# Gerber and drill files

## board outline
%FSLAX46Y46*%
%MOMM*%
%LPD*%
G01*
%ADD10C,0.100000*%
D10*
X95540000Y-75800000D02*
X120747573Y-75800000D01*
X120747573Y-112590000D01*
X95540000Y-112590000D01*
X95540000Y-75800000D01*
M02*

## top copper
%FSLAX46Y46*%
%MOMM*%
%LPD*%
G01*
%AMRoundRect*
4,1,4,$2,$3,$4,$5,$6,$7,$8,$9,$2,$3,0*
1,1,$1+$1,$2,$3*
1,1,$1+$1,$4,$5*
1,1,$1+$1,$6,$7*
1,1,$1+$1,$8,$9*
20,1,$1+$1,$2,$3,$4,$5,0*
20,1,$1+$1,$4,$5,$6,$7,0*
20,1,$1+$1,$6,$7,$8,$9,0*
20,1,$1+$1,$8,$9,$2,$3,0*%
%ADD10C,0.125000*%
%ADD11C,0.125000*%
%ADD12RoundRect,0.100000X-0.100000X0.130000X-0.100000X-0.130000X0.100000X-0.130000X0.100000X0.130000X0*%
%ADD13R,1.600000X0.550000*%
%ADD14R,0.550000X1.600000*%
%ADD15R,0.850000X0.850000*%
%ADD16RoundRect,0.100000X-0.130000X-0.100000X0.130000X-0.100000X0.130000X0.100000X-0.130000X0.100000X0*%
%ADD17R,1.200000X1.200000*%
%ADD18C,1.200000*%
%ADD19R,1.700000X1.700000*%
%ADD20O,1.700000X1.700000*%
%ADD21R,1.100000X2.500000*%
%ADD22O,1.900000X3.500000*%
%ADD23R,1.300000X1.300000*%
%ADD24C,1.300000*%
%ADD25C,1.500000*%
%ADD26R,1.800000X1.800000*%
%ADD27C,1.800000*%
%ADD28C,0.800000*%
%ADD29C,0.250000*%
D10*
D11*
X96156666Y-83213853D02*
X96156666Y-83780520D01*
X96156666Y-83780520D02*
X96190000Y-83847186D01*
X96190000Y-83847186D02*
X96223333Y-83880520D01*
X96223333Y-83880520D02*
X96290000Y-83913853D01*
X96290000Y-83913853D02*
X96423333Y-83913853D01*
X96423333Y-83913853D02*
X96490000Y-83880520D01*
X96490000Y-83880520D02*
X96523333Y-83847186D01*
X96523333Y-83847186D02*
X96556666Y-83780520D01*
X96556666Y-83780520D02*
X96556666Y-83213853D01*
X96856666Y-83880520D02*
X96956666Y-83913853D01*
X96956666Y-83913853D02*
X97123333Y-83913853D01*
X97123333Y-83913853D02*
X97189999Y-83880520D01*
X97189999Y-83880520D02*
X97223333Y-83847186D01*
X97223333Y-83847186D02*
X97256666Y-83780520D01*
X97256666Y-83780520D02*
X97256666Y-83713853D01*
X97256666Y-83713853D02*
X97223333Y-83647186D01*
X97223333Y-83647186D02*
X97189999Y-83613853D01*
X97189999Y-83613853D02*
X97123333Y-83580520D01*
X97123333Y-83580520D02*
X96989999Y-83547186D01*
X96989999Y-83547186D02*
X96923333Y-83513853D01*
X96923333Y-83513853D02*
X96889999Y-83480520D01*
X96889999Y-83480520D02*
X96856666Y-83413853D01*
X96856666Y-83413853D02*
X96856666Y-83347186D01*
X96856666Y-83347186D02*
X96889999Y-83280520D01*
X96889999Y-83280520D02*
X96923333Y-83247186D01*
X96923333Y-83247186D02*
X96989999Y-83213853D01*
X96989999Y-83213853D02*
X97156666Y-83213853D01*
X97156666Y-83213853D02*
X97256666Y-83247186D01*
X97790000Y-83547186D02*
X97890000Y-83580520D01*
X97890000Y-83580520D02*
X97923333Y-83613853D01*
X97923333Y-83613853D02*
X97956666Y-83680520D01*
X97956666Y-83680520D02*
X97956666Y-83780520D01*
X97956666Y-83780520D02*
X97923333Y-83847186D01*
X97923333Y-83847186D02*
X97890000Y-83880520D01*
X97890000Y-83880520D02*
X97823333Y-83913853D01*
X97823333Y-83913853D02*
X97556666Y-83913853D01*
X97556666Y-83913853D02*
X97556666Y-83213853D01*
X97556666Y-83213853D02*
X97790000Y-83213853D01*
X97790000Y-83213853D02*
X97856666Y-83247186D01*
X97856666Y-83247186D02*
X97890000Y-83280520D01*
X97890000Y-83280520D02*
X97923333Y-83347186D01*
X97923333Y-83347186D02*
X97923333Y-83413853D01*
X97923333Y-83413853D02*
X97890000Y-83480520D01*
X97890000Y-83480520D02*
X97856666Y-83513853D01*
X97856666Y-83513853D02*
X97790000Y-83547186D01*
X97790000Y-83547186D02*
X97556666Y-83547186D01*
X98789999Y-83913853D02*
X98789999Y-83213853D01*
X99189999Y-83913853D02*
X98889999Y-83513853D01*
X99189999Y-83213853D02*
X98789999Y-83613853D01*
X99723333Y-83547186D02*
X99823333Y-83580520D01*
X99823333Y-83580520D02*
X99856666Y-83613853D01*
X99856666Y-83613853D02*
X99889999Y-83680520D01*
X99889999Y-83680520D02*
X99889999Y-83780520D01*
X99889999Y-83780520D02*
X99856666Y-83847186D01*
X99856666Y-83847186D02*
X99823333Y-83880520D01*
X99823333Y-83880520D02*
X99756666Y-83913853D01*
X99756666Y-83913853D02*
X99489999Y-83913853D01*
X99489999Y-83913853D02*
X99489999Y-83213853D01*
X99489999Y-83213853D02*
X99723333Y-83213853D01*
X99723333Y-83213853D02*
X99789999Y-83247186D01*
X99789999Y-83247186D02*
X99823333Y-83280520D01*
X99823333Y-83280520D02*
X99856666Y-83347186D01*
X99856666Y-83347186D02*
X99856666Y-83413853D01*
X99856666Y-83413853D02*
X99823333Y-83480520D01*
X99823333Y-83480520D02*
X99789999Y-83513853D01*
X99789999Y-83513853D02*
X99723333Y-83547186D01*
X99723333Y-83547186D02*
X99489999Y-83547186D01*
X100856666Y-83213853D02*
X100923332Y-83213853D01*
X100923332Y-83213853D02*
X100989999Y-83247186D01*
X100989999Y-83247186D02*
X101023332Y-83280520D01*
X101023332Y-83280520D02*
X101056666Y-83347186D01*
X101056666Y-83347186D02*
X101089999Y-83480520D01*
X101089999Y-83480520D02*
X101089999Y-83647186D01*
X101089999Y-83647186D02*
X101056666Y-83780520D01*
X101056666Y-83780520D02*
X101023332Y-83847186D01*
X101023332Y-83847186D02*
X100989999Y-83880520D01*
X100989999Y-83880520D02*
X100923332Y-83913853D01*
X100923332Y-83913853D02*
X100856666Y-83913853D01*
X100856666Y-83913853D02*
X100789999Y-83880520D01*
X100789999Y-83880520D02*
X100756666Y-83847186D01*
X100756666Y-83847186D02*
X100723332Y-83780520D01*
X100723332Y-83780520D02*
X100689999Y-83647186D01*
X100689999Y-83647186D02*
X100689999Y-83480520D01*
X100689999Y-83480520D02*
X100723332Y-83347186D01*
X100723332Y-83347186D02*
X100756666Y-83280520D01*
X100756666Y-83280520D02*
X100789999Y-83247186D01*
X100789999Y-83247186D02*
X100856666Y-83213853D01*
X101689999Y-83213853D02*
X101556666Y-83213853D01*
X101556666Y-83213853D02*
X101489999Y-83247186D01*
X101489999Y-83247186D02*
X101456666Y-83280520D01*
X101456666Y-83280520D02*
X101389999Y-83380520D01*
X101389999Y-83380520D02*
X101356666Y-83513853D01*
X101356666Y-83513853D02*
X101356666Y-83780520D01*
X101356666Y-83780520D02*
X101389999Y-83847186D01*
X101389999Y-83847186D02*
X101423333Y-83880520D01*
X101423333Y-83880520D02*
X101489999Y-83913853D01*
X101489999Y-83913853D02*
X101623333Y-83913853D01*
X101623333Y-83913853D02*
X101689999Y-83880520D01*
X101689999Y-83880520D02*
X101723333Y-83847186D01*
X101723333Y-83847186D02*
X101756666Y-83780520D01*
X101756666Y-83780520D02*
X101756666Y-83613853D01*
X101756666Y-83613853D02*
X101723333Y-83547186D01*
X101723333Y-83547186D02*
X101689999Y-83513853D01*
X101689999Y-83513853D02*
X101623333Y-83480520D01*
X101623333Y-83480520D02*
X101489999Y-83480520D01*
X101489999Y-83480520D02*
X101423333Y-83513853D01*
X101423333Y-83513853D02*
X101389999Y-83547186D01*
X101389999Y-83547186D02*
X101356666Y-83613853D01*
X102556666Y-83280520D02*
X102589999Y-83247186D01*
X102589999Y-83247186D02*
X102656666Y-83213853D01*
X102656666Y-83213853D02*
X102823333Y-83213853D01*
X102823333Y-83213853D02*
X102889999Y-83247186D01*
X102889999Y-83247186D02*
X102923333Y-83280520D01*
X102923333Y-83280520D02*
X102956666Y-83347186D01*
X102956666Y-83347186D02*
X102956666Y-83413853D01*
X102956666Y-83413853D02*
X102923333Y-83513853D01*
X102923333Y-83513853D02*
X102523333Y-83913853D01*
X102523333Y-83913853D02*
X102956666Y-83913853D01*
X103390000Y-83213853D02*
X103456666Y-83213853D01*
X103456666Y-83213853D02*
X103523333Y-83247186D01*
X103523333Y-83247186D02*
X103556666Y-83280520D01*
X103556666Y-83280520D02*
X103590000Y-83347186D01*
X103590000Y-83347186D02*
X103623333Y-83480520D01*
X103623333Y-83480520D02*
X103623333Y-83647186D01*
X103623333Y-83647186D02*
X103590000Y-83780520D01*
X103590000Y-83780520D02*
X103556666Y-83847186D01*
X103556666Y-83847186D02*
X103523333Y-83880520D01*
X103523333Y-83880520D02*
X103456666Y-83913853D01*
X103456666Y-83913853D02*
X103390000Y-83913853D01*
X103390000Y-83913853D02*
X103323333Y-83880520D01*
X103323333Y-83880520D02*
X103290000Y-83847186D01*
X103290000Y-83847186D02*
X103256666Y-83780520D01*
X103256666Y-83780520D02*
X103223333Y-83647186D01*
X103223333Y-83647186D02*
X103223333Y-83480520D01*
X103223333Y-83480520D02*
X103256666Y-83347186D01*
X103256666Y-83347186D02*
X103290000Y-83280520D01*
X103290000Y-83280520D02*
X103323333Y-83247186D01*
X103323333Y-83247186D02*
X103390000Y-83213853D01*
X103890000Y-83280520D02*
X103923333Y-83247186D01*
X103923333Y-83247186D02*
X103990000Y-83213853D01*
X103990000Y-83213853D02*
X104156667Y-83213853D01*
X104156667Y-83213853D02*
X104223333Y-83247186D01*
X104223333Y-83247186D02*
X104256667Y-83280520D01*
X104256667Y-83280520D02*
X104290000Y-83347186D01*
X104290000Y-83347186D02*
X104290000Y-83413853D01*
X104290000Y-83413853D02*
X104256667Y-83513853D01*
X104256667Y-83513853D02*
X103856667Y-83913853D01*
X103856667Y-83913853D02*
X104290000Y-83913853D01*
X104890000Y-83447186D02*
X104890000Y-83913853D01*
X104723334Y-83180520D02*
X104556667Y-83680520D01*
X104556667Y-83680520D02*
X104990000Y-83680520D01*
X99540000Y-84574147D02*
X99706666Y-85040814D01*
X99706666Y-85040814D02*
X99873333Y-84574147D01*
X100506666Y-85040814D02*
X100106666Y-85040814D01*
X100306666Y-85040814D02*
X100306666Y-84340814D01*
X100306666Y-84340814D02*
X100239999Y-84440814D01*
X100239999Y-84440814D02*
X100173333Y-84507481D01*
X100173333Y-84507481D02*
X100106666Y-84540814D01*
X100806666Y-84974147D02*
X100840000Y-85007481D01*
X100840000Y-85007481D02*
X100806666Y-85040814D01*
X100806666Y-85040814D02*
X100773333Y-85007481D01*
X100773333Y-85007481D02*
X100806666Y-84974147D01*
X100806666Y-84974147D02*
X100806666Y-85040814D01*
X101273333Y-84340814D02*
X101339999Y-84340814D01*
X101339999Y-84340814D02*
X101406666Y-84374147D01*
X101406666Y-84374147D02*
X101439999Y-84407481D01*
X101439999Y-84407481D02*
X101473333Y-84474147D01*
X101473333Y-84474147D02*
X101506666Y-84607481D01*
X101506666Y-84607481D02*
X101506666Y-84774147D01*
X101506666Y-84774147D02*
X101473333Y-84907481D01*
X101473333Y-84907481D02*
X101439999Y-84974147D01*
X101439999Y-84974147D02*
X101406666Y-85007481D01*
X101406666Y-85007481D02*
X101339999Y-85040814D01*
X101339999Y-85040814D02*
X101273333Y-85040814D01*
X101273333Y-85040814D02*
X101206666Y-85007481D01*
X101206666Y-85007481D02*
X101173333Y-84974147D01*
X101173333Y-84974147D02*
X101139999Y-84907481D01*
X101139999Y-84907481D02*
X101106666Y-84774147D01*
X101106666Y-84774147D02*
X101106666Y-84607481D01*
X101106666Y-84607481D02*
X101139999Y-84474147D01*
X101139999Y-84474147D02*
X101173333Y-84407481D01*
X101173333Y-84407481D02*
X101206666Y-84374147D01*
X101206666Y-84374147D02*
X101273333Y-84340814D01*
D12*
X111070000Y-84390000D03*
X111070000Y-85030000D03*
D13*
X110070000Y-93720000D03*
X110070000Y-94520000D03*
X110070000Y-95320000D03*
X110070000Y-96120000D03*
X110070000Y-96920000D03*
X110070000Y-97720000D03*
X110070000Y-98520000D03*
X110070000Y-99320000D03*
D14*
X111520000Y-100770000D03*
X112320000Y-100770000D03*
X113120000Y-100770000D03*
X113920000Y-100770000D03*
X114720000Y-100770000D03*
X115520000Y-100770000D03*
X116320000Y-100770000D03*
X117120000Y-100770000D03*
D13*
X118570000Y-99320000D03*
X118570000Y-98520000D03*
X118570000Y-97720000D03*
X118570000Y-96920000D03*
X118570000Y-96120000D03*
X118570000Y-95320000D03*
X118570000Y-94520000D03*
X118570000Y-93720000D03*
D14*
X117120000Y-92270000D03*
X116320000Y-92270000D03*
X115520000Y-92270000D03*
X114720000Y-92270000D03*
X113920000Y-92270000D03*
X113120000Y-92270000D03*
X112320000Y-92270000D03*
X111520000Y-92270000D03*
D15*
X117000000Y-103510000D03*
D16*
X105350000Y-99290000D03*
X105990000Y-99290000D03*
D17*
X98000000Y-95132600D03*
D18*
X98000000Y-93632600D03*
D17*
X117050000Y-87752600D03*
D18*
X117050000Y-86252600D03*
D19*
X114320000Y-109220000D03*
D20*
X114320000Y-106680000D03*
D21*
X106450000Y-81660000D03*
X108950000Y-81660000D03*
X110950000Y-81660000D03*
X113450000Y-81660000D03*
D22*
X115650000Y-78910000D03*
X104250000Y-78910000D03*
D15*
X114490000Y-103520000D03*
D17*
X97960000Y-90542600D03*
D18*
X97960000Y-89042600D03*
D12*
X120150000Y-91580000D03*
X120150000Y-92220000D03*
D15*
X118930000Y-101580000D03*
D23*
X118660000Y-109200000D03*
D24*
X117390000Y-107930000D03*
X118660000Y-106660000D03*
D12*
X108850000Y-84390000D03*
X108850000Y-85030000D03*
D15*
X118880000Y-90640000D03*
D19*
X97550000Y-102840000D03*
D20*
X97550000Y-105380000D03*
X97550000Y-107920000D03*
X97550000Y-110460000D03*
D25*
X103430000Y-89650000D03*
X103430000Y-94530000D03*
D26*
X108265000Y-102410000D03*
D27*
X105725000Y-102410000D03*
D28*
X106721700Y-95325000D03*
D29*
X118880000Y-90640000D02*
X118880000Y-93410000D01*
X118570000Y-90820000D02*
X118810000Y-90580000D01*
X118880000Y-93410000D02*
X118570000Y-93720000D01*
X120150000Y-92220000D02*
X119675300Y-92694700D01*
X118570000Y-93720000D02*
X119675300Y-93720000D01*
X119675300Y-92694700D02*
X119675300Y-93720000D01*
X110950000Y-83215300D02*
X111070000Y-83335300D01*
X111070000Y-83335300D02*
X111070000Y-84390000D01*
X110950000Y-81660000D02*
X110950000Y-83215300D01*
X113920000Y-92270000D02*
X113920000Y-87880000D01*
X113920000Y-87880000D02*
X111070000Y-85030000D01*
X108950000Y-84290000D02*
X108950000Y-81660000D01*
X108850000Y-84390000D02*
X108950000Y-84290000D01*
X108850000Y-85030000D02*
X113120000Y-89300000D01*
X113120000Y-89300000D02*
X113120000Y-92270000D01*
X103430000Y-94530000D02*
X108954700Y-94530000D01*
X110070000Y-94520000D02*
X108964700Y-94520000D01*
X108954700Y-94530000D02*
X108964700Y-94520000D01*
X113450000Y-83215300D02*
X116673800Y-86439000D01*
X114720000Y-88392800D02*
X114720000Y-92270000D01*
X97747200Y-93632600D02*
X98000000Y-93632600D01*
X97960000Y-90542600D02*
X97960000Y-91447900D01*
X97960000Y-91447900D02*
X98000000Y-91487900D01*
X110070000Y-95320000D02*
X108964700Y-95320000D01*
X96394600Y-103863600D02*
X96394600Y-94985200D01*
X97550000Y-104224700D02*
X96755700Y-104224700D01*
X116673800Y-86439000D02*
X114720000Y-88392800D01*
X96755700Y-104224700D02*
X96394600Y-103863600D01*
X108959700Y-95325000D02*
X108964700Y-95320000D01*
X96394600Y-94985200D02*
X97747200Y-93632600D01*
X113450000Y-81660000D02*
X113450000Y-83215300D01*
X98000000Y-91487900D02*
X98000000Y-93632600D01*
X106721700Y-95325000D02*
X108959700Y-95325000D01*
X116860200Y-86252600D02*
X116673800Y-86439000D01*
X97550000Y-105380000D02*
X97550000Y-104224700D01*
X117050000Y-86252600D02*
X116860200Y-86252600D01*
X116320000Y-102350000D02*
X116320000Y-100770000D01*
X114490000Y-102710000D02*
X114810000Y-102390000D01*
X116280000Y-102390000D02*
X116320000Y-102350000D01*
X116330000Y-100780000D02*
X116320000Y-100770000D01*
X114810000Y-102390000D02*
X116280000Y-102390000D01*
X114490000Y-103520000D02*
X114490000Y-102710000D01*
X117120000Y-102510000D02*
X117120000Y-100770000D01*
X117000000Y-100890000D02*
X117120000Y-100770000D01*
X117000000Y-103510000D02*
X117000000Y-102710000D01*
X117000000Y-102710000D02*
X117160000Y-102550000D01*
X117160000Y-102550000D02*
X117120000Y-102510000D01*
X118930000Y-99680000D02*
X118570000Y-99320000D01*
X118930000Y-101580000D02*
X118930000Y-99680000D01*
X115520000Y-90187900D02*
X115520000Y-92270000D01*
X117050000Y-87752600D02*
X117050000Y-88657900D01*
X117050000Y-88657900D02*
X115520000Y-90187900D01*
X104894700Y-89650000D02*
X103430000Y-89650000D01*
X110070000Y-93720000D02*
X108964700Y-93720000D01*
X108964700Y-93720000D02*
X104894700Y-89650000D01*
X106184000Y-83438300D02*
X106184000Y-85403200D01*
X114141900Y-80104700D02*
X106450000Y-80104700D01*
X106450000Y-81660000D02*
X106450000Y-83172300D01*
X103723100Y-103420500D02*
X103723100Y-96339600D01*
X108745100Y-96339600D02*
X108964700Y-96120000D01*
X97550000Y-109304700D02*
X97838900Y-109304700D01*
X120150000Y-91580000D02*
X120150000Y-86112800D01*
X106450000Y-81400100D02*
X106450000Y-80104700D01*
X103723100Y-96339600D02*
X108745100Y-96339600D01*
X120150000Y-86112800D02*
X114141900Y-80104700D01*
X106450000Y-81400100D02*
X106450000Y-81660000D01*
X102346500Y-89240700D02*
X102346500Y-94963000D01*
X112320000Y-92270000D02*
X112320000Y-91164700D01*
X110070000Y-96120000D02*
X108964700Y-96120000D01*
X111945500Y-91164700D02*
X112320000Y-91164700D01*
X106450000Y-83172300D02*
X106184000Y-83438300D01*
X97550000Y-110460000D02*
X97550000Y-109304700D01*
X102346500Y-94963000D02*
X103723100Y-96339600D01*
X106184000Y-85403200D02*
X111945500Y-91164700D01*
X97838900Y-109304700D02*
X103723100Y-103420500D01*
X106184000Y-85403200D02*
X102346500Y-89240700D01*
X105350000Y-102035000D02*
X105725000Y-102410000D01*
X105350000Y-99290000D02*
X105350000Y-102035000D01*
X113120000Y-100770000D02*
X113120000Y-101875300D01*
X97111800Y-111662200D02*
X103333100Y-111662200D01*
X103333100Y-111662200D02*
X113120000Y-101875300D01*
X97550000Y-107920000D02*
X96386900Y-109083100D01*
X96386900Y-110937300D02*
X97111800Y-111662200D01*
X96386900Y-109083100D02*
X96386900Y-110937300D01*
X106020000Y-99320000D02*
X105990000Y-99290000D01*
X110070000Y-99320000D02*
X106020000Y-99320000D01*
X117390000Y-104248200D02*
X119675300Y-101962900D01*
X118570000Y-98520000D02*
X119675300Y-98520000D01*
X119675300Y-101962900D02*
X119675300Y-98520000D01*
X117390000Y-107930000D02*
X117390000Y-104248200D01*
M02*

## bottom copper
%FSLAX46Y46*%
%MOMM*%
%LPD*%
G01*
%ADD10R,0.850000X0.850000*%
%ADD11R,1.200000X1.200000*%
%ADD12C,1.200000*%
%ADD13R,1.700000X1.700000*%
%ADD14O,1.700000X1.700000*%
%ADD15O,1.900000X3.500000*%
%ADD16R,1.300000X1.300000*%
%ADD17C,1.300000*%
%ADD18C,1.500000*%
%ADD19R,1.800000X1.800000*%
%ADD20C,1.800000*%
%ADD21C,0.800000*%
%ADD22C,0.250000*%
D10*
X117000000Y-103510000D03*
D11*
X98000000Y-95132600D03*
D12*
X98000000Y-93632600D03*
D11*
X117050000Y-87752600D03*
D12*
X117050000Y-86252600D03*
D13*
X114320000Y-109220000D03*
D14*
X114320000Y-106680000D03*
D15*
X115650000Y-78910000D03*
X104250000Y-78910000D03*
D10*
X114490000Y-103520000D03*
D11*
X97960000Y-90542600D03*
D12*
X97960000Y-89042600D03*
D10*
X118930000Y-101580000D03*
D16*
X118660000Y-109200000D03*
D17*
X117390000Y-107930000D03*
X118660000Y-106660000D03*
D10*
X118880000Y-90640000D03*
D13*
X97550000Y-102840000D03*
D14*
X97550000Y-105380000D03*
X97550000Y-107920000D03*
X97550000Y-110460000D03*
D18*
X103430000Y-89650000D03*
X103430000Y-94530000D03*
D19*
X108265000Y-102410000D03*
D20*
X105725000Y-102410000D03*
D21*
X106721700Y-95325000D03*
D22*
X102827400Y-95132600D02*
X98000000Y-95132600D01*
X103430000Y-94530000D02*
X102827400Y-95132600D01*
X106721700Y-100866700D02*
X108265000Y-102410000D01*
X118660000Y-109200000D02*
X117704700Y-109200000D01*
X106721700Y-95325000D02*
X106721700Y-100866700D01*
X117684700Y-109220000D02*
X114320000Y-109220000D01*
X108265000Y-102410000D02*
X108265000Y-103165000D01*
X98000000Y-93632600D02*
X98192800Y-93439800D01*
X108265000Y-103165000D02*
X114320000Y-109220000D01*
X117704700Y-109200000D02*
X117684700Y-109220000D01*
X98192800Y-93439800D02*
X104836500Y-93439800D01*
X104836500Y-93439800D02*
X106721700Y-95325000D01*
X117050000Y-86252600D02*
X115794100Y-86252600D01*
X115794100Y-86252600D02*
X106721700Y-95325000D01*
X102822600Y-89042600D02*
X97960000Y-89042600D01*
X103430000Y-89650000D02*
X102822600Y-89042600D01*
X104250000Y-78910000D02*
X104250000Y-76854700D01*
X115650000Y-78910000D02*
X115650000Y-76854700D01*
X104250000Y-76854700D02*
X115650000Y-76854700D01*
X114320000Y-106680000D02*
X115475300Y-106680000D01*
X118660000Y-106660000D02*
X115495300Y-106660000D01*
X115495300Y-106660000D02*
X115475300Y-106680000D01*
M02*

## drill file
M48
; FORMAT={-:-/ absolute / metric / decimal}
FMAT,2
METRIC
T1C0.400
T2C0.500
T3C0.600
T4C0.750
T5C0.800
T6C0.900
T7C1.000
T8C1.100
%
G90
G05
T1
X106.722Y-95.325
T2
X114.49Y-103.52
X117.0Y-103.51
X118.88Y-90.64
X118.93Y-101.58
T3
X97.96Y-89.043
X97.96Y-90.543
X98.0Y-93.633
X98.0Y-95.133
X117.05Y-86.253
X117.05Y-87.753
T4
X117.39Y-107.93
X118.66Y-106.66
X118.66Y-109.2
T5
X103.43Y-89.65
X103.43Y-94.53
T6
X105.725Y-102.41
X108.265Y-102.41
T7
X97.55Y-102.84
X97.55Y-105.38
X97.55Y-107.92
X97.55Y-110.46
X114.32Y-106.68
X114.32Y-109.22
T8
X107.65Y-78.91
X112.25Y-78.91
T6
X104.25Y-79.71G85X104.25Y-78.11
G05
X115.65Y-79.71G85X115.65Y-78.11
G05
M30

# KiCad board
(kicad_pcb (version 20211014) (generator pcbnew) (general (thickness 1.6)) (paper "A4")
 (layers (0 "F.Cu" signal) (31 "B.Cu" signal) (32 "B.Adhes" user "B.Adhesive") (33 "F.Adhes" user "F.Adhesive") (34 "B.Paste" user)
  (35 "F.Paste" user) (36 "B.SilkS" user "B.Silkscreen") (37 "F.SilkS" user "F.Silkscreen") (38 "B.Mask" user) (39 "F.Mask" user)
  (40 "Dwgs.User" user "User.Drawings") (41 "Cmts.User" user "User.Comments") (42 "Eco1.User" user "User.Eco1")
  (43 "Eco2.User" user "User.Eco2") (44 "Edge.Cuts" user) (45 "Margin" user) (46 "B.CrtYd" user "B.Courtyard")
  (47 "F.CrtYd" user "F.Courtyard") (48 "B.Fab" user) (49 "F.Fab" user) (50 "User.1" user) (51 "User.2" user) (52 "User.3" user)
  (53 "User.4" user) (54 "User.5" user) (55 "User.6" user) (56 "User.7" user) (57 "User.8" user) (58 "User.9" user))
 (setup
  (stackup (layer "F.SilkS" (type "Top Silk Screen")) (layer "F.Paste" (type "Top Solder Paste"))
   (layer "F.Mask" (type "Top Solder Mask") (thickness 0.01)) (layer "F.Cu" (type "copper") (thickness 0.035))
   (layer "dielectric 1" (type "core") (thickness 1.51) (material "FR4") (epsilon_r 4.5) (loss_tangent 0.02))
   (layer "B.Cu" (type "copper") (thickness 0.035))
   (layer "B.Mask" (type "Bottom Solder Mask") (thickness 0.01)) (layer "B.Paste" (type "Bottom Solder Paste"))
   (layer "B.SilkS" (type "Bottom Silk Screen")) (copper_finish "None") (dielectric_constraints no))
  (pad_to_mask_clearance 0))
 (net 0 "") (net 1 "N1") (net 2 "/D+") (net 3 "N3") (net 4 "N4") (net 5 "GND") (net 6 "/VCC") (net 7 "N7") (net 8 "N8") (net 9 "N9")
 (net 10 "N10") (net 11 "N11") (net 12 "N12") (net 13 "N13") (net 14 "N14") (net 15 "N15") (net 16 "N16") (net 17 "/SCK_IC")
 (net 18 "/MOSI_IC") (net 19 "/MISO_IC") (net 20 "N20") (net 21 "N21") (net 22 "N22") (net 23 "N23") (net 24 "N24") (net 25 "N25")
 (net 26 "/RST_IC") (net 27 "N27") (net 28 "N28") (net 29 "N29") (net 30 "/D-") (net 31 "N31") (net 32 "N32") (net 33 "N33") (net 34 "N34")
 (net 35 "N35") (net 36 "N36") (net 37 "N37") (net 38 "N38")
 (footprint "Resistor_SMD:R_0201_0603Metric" (layer "F.Cu") (at 111.07 84.71 -90)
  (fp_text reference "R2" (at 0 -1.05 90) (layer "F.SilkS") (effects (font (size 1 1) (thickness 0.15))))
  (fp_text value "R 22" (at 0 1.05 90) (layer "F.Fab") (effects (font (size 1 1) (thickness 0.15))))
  (pad "" smd roundrect (at 0.345 0 270) (size 0.318 0.36) (layers "F.Paste") (roundrect_rratio 0.25))
  (pad "" smd roundrect (at -0.345 0 270) (size 0.318 0.36) (layers "F.Paste") (roundrect_rratio 0.25))
  (pad "1" smd roundrect (at -0.32 0 270) (size 0.46 0.4) (layers "F.Cu" "F.Mask") (roundrect_rratio 0.25) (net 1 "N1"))
  (pad "2" smd roundrect (at 0.32 0 270) (size 0.46 0.4) (layers "F.Cu" "F.Mask") (roundrect_rratio 0.25) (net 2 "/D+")))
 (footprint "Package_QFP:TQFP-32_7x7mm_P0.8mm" (layer "F.Cu") (at 114.32 96.52)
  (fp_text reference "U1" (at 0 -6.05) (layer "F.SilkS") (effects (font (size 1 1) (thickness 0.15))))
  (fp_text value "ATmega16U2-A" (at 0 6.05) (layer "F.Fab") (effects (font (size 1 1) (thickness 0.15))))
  (pad "1" smd rect (at -4.25 -2.8) (size 1.6 0.55) (layers "F.Cu" "F.Paste" "F.Mask") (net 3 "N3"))
  (pad "2" smd rect (at -4.25 -2) (size 1.6 0.55) (layers "F.Cu" "F.Paste" "F.Mask") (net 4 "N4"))
  (pad "3" smd rect (at -4.25 -1.2) (size 1.6 0.55) (layers "F.Cu" "F.Paste" "F.Mask") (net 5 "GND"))
  (pad "4" smd rect (at -4.25 -0.4) (size 1.6 0.55) (layers "F.Cu" "F.Paste" "F.Mask") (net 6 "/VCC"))
  (pad "5" smd rect (at -4.25 0.4) (size 1.6 0.55) (layers "F.Cu" "F.Paste" "F.Mask") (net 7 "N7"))
  (pad "6" smd rect (at -4.25 1.2) (size 1.6 0.55) (layers "F.Cu" "F.Paste" "F.Mask") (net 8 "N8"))
  (pad "7" smd rect (at -4.25 2) (size 1.6 0.55) (layers "F.Cu" "F.Paste" "F.Mask") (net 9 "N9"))
  (pad "8" smd rect (at -4.25 2.8) (size 1.6 0.55) (layers "F.Cu" "F.Paste" "F.Mask") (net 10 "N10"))
  (pad "9" smd rect (at -2.8 4.25 90) (size 1.6 0.55) (layers "F.Cu" "F.Paste" "F.Mask") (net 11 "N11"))
  (pad "10" smd rect (at -2 4.25 90) (size 1.6 0.55) (layers "F.Cu" "F.Paste" "F.Mask") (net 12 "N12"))
  (pad "11" smd rect (at -1.2 4.25 90) (size 1.6 0.55) (layers "F.Cu" "F.Paste" "F.Mask") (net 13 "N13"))
  (pad "12" smd rect (at -0.4 4.25 90) (size 1.6 0.55) (layers "F.Cu" "F.Paste" "F.Mask") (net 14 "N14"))
  (pad "13" smd rect (at 0.4 4.25 90) (size 1.6 0.55) (layers "F.Cu" "F.Paste" "F.Mask") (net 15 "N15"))
  (pad "14" smd rect (at 1.2 4.25 90) (size 1.6 0.55) (layers "F.Cu" "F.Paste" "F.Mask") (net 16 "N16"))
  (pad "15" smd rect (at 2 4.25 90) (size 1.6 0.55) (layers "F.Cu" "F.Paste" "F.Mask") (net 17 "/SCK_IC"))
  (pad "16" smd rect (at 2.8 4.25 90) (size 1.6 0.55) (layers "F.Cu" "F.Paste" "F.Mask") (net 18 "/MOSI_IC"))
  (pad "17" smd rect (at 4.25 2.8) (size 1.6 0.55) (layers "F.Cu" "F.Paste" "F.Mask") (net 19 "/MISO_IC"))
  (pad "18" smd rect (at 4.25 2) (size 1.6 0.55) (layers "F.Cu" "F.Paste" "F.Mask") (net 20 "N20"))
  (pad "19" smd rect (at 4.25 1.2) (size 1.6 0.55) (layers "F.Cu" "F.Paste" "F.Mask") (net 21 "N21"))
  (pad "20" smd rect (at 4.25 0.4) (size 1.6 0.55) (layers "F.Cu" "F.Paste" "F.Mask") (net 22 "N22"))
  (pad "21" smd rect (at 4.25 -0.4) (size 1.6 0.55) (layers "F.Cu" "F.Paste" "F.Mask") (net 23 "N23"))
  (pad "22" smd rect (at 4.25 -1.2) (size 1.6 0.55) (layers "F.Cu" "F.Paste" "F.Mask") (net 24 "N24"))
  (pad "23" smd rect (at 4.25 -2) (size 1.6 0.55) (layers "F.Cu" "F.Paste" "F.Mask") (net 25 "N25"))
  (pad "24" smd rect (at 4.25 -2.8) (size 1.6 0.55) (layers "F.Cu" "F.Paste" "F.Mask") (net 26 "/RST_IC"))
  (pad "25" smd rect (at 2.8 -4.25 90) (size 1.6 0.55) (layers "F.Cu" "F.Paste" "F.Mask") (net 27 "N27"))
  (pad "26" smd rect (at 2 -4.25 90) (size 1.6 0.55) (layers "F.Cu" "F.Paste" "F.Mask") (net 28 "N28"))
  (pad "27" smd rect (at 1.2 -4.25 90) (size 1.6 0.55) (layers "F.Cu" "F.Paste" "F.Mask") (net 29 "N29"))
  (pad "28" smd rect (at 0.4 -4.25 90) (size 1.6 0.55) (layers "F.Cu" "F.Paste" "F.Mask") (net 5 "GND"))
  (pad "29" smd rect (at -0.4 -4.25 90) (size 1.6 0.55) (layers "F.Cu" "F.Paste" "F.Mask") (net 2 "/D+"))
  (pad "30" smd rect (at -1.2 -4.25 90) (size 1.6 0.55) (layers "F.Cu" "F.Paste" "F.Mask") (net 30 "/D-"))
  (pad "31" smd rect (at -2 -4.25 90) (size 1.6 0.55) (layers "F.Cu" "F.Paste" "F.Mask") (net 6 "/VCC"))
  (pad "32" smd rect (at -2.8 -4.25 90) (size 1.6 0.55) (layers "F.Cu" "F.Paste" "F.Mask") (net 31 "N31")))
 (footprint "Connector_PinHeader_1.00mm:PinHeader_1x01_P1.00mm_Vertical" (layer "F.Cu") (at 117 103.51)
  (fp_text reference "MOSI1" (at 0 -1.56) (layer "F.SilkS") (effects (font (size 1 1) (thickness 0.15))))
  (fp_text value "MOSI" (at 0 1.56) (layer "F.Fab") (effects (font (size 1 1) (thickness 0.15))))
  (pad "1" thru_hole rect (at 0 0) (size 0.85 0.85) (drill 0.5) (layers *.Cu *.Mask) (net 18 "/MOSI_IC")))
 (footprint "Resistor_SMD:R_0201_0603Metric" (layer "F.Cu") (at 105.67 99.29)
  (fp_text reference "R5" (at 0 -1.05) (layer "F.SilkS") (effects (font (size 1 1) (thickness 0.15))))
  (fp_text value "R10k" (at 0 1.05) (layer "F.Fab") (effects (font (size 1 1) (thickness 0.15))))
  (pad "" smd roundrect (at 0.345 0) (size 0.318 0.36) (layers "F.Paste") (roundrect_rratio 0.25))
  (pad "" smd roundrect (at -0.345 0) (size 0.318 0.36) (layers "F.Paste") (roundrect_rratio 0.25))
  (pad "1" smd roundrect (at -0.32 0) (size 0.46 0.4) (layers "F.Cu" "F.Mask") (roundrect_rratio 0.25) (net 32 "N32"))
  (pad "2" smd roundrect (at 0.32 0) (size 0.46 0.4) (layers "F.Cu" "F.Mask") (roundrect_rratio 0.25) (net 10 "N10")))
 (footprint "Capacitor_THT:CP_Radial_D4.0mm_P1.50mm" (layer "F.Cu") (at 98 95.1326 90)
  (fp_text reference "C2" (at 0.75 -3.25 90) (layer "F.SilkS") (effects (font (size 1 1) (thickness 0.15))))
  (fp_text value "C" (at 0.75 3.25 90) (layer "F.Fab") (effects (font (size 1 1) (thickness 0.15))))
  (pad "1" thru_hole rect (at 0 0 90) (size 1.2 1.2) (drill 0.6) (layers *.Cu *.Mask) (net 4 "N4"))
  (pad "2" thru_hole circle (at 1.5 0 90) (size 1.2 1.2) (drill 0.6) (layers *.Cu *.Mask) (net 5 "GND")))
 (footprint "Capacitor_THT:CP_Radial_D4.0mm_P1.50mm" (layer "F.Cu") (at 117.05 87.7526 90)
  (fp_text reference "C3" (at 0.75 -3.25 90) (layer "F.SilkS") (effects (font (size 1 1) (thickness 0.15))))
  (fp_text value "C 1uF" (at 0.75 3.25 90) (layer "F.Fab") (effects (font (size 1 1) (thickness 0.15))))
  (pad "1" thru_hole rect (at 0 0 90) (size 1.2 1.2) (drill 0.6) (layers *.Cu *.Mask) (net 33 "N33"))
  (pad "2" thru_hole circle (at 1.5 0 90) (size 1.2 1.2) (drill 0.6) (layers *.Cu *.Mask) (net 5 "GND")))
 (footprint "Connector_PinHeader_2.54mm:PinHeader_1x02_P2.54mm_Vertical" (layer "F.Cu") (at 114.32 109.22 180)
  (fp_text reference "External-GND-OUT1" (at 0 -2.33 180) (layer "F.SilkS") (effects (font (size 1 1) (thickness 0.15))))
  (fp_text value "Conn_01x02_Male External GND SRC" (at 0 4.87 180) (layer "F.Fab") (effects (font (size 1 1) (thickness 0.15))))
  (pad "1" thru_hole rect (at 0 0 180) (size 1.7 1.7) (drill 1) (layers *.Cu *.Mask) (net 5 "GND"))
  (pad "2" thru_hole oval (at 0 2.54 180) (size 1.7 1.7) (drill 1) (layers *.Cu *.Mask) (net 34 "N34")))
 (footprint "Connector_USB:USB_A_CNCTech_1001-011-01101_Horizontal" (layer "F.Cu") (at 109.95 72.01 90)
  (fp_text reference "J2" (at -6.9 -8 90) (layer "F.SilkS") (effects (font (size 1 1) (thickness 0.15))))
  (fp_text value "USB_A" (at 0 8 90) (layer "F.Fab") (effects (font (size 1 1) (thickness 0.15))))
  (pad "" np_thru_hole circle (at -6.9 2.3 90) (size 1.1 1.1) (drill 1.1) (layers *.Cu *.Mask))
  (pad "" np_thru_hole circle (at -6.9 -2.3 90) (size 1.1 1.1) (drill 1.1) (layers *.Cu *.Mask))
  (pad "1" smd rect (at -9.65 -3.5 90) (size 2.5 1.1) (layers "F.Cu" "F.Paste" "F.Mask") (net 6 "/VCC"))
  (pad "2" smd rect (at -9.65 -1 90) (size 2.5 1.1) (layers "F.Cu" "F.Paste" "F.Mask") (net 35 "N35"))
  (pad "3" smd rect (at -9.65 1 90) (size 2.5 1.1) (layers "F.Cu" "F.Paste" "F.Mask") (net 1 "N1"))
  (pad "4" smd rect (at -9.65 3.5 90) (size 2.5 1.1) (layers "F.Cu" "F.Paste" "F.Mask") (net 5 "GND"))
  (pad "5" thru_hole oval (at -6.9 5.7 90) (size 3.5 1.9) (drill oval 2.5 0.9) (layers *.Cu *.Mask) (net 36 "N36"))
  (pad "5" thru_hole oval (at -6.9 -5.7 90) (size 3.5 1.9) (drill oval 2.5 0.9) (layers *.Cu *.Mask) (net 36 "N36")))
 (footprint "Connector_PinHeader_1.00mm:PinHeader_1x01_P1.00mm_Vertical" (layer "F.Cu") (at 114.49 103.52)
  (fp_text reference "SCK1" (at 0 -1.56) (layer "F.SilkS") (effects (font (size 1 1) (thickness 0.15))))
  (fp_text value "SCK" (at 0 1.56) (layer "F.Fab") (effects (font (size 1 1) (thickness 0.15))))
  (pad "1" thru_hole rect (at 0 0) (size 0.85 0.85) (drill 0.5) (layers *.Cu *.Mask) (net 17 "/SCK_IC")))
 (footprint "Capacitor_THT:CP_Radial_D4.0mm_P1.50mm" (layer "F.Cu") (at 97.96 90.5426 90)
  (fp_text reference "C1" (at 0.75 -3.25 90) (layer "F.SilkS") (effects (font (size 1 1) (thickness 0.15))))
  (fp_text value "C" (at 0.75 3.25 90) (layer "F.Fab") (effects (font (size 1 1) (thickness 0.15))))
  (pad "1" thru_hole rect (at 0 0 90) (size 1.2 1.2) (drill 0.6) (layers *.Cu *.Mask) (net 5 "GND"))
  (pad "2" thru_hole circle (at 1.5 0 90) (size 1.2 1.2) (drill 0.6) (layers *.Cu *.Mask) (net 3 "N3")))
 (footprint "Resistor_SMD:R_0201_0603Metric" (layer "F.Cu") (at 120.15 91.9 -90)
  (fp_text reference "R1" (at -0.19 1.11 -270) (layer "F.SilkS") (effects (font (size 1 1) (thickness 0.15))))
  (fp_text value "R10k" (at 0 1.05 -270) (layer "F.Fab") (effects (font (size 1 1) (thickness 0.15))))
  (pad "" smd roundrect (at -0.345 0 270) (size 0.318 0.36) (layers "F.Paste") (roundrect_rratio 0.25))
  (pad "" smd roundrect (at 0.345 0 270) (size 0.318 0.36) (layers "F.Paste") (roundrect_rratio 0.25))
  (pad "1" smd roundrect (at -0.32 0 270) (size 0.46 0.4) (layers "F.Cu" "F.Mask") (roundrect_rratio 0.25) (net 6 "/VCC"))
  (pad "2" smd roundrect (at 0.32 0 270) (size 0.46 0.4) (layers "F.Cu" "F.Mask") (roundrect_rratio 0.25) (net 26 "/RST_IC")))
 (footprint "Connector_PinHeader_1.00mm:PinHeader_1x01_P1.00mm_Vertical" (layer "F.Cu") (at 118.93 101.58)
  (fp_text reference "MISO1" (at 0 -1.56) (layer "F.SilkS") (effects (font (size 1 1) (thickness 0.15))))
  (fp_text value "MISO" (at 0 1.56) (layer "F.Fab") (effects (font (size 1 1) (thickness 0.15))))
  (pad "1" thru_hole rect (at 0 0) (size 0.85 0.85) (drill 0.5) (layers *.Cu *.Mask) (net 19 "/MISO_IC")))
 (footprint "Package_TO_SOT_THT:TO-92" (layer "F.Cu") (at 118.66 109.2 90)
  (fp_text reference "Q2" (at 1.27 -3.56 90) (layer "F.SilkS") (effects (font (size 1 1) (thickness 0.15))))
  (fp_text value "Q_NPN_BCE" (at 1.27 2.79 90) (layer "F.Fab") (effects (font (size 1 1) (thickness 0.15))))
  (pad "1" thru_hole rect (at 0 0 90) (size 1.3 1.3) (drill 0.75) (layers *.Cu *.Mask) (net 5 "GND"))
  (pad "2" thru_hole circle (at 1.27 -1.27 90) (size 1.3 1.3) (drill 0.75) (layers *.Cu *.Mask) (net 20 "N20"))
  (pad "3" thru_hole circle (at 2.54 0 90) (size 1.3 1.3) (drill 0.75) (layers *.Cu *.Mask) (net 34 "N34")))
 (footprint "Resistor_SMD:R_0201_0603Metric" (layer "F.Cu") (at 108.85 84.71 -90)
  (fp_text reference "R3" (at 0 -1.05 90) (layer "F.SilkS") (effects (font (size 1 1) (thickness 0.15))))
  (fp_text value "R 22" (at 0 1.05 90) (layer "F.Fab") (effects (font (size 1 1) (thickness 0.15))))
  (pad "" smd roundrect (at -0.345 0 270) (size 0.318 0.36) (layers "F.Paste") (roundrect_rratio 0.25))
  (pad "" smd roundrect (at 0.345 0 270) (size 0.318 0.36) (layers "F.Paste") (roundrect_rratio 0.25))
  (pad "1" smd roundrect (at -0.32 0 270) (size 0.46 0.4) (layers "F.Cu" "F.Mask") (roundrect_rratio 0.25) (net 35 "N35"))
  (pad "2" smd roundrect (at 0.32 0 270) (size 0.46 0.4) (layers "F.Cu" "F.Mask") (roundrect_rratio 0.25) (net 30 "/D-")))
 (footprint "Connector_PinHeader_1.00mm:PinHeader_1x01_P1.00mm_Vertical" (layer "F.Cu") (at 118.88 90.64)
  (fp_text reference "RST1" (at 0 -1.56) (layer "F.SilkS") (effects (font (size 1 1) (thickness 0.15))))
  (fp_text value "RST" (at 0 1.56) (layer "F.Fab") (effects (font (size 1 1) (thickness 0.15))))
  (pad "1" thru_hole rect (at 0 0) (size 0.85 0.85) (drill 0.5) (layers *.Cu *.Mask) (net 26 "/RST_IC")))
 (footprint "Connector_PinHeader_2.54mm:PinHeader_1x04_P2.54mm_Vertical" (layer "F.Cu") (at 97.55 102.84)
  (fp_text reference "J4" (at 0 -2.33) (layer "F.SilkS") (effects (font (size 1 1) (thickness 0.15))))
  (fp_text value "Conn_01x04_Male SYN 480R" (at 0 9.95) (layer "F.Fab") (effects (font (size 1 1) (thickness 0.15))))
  (pad "1" thru_hole rect (at 0 0) (size 1.7 1.7) (drill 1) (layers *.Cu *.Mask) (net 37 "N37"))
  (pad "2" thru_hole oval (at 0 2.54) (size 1.7 1.7) (drill 1) (layers *.Cu *.Mask) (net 5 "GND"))
  (pad "3" thru_hole oval (at 0 5.08) (size 1.7 1.7) (drill 1) (layers *.Cu *.Mask) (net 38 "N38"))
  (pad "4" thru_hole oval (at 0 7.62) (size 1.7 1.7) (drill 1) (layers *.Cu *.Mask) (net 6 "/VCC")))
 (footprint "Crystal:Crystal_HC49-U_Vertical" (layer "F.Cu") (at 103.43 89.65 -90)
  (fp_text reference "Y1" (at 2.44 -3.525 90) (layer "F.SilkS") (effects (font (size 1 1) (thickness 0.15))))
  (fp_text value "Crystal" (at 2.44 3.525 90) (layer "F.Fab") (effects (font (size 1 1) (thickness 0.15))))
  (pad "1" thru_hole circle (at 0 0 270) (size 1.5 1.5) (drill 0.8) (layers *.Cu *.Mask) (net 3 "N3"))
  (pad "2" thru_hole circle (at 4.88 0 270) (size 1.5 1.5) (drill 0.8) (layers *.Cu *.Mask) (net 4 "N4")))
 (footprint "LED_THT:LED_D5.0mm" (layer "F.Cu") (at 108.265 102.41 180)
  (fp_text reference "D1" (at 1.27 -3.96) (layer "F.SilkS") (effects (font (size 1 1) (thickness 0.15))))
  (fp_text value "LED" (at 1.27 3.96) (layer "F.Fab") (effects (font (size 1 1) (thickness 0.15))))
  (pad "1" thru_hole rect (at 0 0 180) (size 1.8 1.8) (drill 0.9) (layers *.Cu *.Mask) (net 5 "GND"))
  (pad "2" thru_hole circle (at 2.54 0 180) (size 1.8 1.8) (drill 0.9) (layers *.Cu *.Mask) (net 32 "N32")))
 (gr_rect (start 120.747573 75.8) (end 95.54 112.59) (layer "Edge.Cuts") (width 0.1) (fill none))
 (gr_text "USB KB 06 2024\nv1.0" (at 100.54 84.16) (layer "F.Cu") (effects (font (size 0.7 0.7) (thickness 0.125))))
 (segment (start 118.88 90.64) (end 118.88 93.41) (width 0.25) (layer "F.Cu") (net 26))
 (segment (start 118.57 90.82) (end 118.81 90.58) (width 0.25) (layer "F.Cu") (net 26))
 (segment (start 118.88 93.41) (end 118.57 93.72) (width 0.25) (layer "F.Cu") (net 26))
 (segment (start 120.15 92.22) (end 119.6753 92.6947) (width 0.25) (layer "F.Cu") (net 26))
 (segment (start 118.57 93.72) (end 119.6753 93.72) (width 0.25) (layer "F.Cu") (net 26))
 (segment (start 119.6753 92.6947) (end 119.6753 93.72) (width 0.25) (layer "F.Cu") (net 26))
 (segment (start 110.95 83.2153) (end 111.07 83.3353) (width 0.25) (layer "F.Cu") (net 1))
 (segment (start 111.07 83.3353) (end 111.07 84.39) (width 0.25) (layer "F.Cu") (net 1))
 (segment (start 110.95 81.66) (end 110.95 83.2153) (width 0.25) (layer "F.Cu") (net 1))
 (segment (start 113.92 92.27) (end 113.92 87.88) (width 0.25) (layer "F.Cu") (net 2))
 (segment (start 113.92 87.88) (end 111.07 85.03) (width 0.25) (layer "F.Cu") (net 2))
 (segment (start 108.95 84.29) (end 108.95 81.66) (width 0.25) (layer "F.Cu") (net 35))
 (segment (start 108.85 84.39) (end 108.95 84.29) (width 0.25) (layer "F.Cu") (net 35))
 (segment (start 108.85 85.03) (end 113.12 89.3) (width 0.25) (layer "F.Cu") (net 30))
 (segment (start 113.12 89.3) (end 113.12 92.27) (width 0.25) (layer "F.Cu") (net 30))
 (segment (start 103.43 94.53) (end 108.9547 94.53) (width 0.25) (layer "F.Cu") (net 4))
 (segment (start 110.07 94.52) (end 108.9647 94.52) (width 0.25) (layer "F.Cu") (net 4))
 (segment (start 108.9547 94.53) (end 108.9647 94.52) (width 0.25) (layer "F.Cu") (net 4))
 (segment (start 102.8274 95.1326) (end 98 95.1326) (width 0.25) (layer "B.Cu") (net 4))
 (segment (start 103.43 94.53) (end 102.8274 95.1326) (width 0.25) (layer "B.Cu") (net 4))
 (segment (start 113.45 83.2153) (end 116.6738 86.439) (width 0.25) (layer "F.Cu") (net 5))
 (segment (start 114.72 88.3928) (end 114.72 92.27) (width 0.25) (layer "F.Cu") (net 5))
 (segment (start 97.7472 93.6326) (end 98 93.6326) (width 0.25) (layer "F.Cu") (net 5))
 (segment (start 97.96 90.5426) (end 97.96 91.4479) (width 0.25) (layer "F.Cu") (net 5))
 (segment (start 97.96 91.4479) (end 98 91.4879) (width 0.25) (layer "F.Cu") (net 5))
 (segment (start 110.07 95.32) (end 108.9647 95.32) (width 0.25) (layer "F.Cu") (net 5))
 (segment (start 96.3946 103.8636) (end 96.3946 94.9852) (width 0.25) (layer "F.Cu") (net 5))
 (segment (start 97.55 104.2247) (end 96.7557 104.2247) (width 0.25) (layer "F.Cu") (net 5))
 (segment (start 116.6738 86.439) (end 114.72 88.3928) (width 0.25) (layer "F.Cu") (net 5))
 (segment (start 96.7557 104.2247) (end 96.3946 103.8636) (width 0.25) (layer "F.Cu") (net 5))
 (segment (start 108.9597 95.325) (end 108.9647 95.32) (width 0.25) (layer "F.Cu") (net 5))
 (segment (start 96.3946 94.9852) (end 97.7472 93.6326) (width 0.25) (layer "F.Cu") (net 5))
 (segment (start 113.45 81.66) (end 113.45 83.2153) (width 0.25) (layer "F.Cu") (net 5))
 (segment (start 98 91.4879) (end 98 93.6326) (width 0.25) (layer "F.Cu") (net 5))
 (segment (start 106.7217 95.325) (end 108.9597 95.325) (width 0.25) (layer "F.Cu") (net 5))
 (segment (start 116.8602 86.2526) (end 116.6738 86.439) (width 0.25) (layer "F.Cu") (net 5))
 (segment (start 97.55 105.38) (end 97.55 104.2247) (width 0.25) (layer "F.Cu") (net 5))
 (segment (start 117.05 86.2526) (end 116.8602 86.2526) (width 0.25) (layer "F.Cu") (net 5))
 (via (at 106.7217 95.325) (size 0.8) (drill 0.4) (layers "F.Cu" "B.Cu") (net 5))
 (segment (start 106.7217 100.8667) (end 108.265 102.41) (width 0.25) (layer "B.Cu") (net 5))
 (segment (start 118.66 109.2) (end 117.7047 109.2) (width 0.25) (layer "B.Cu") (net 5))
 (segment (start 106.7217 95.325) (end 106.7217 100.8667) (width 0.25) (layer "B.Cu") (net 5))
 (segment (start 117.6847 109.22) (end 114.32 109.22) (width 0.25) (layer "B.Cu") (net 5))
 (segment (start 108.265 102.41) (end 108.265 103.165) (width 0.25) (layer "B.Cu") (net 5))
 (segment (start 98 93.6326) (end 98.1928 93.4398) (width 0.25) (layer "B.Cu") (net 5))
 (segment (start 108.265 103.165) (end 114.32 109.22) (width 0.25) (layer "B.Cu") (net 5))
 (segment (start 117.7047 109.2) (end 117.6847 109.22) (width 0.25) (layer "B.Cu") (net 5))
 (segment (start 98.1928 93.4398) (end 104.8365 93.4398) (width 0.25) (layer "B.Cu") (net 5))
 (segment (start 104.8365 93.4398) (end 106.7217 95.325) (width 0.25) (layer "B.Cu") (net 5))
 (segment (start 117.05 86.2526) (end 115.7941 86.2526) (width 0.25) (layer "B.Cu") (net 5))
 (segment (start 115.7941 86.2526) (end 106.7217 95.325) (width 0.25) (layer "B.Cu") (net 5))
 (segment (start 116.32 102.35) (end 116.32 100.77) (width 0.25) (layer "F.Cu") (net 17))
 (segment (start 114.49 102.71) (end 114.81 102.39) (width 0.25) (layer "F.Cu") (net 17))
 (segment (start 116.28 102.39) (end 116.32 102.35) (width 0.25) (layer "F.Cu") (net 17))
 (segment (start 116.33 100.78) (end 116.32 100.77) (width 0.25) (layer "F.Cu") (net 17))
 (segment (start 114.81 102.39) (end 116.28 102.39) (width 0.25) (layer "F.Cu") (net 17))
 (segment (start 114.49 103.52) (end 114.49 102.71) (width 0.25) (layer "F.Cu") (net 17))
 (segment (start 117.12 102.51) (end 117.12 100.77) (width 0.25) (layer "F.Cu") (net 18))
 (segment (start 117 100.89) (end 117.12 100.77) (width 0.25) (layer "F.Cu") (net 18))
 (segment (start 117 103.51) (end 117 102.71) (width 0.25) (layer "F.Cu") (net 18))
 (segment (start 117 102.71) (end 117.16 102.55) (width 0.25) (layer "F.Cu") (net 18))
 (segment (start 117.16 102.55) (end 117.12 102.51) (width 0.25) (layer "F.Cu") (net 18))
 (segment (start 118.93 99.68) (end 118.57 99.32) (width 0.25) (layer "F.Cu") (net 19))
 (segment (start 118.93 101.58) (end 118.93 99.68) (width 0.25) (layer "F.Cu") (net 19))
 (segment (start 115.52 90.1879) (end 115.52 92.27) (width 0.25) (layer "F.Cu") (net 33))
 (segment (start 117.05 87.7526) (end 117.05 88.6579) (width 0.25) (layer "F.Cu") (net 33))
 (segment (start 117.05 88.6579) (end 115.52 90.1879) (width 0.25) (layer "F.Cu") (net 33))
 (segment (start 104.8947 89.65) (end 103.43 89.65) (width 0.25) (layer "F.Cu") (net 3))
 (segment (start 110.07 93.72) (end 108.9647 93.72) (width 0.25) (layer "F.Cu") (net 3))
 (segment (start 108.9647 93.72) (end 104.8947 89.65) (width 0.25) (layer "F.Cu") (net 3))
 (segment (start 102.8226 89.0426) (end 97.96 89.0426) (width 0.25) (layer "B.Cu") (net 3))
 (segment (start 103.43 89.65) (end 102.8226 89.0426) (width 0.25) (layer "B.Cu") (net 3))
 (segment (start 106.184 83.4383) (end 106.184 85.4032) (width 0.25) (layer "F.Cu") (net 6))
 (segment (start 114.1419 80.1047) (end 106.45 80.1047) (width 0.25) (layer "F.Cu") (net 6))
 (segment (start 106.45 81.66) (end 106.45 83.1723) (width 0.25) (layer "F.Cu") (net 6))
 (segment (start 103.7231 103.4205) (end 103.7231 96.3396) (width 0.25) (layer "F.Cu") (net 6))
 (segment (start 108.7451 96.3396) (end 108.9647 96.12) (width 0.25) (layer "F.Cu") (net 6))
 (segment (start 97.55 109.3047) (end 97.8389 109.3047) (width 0.25) (layer "F.Cu") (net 6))
 (segment (start 120.15 91.58) (end 120.15 86.1128) (width 0.25) (layer "F.Cu") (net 6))
 (segment (start 106.45 81.4001) (end 106.45 80.1047) (width 0.25) (layer "F.Cu") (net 6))
 (segment (start 103.7231 96.3396) (end 108.7451 96.3396) (width 0.25) (layer "F.Cu") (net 6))
 (segment (start 120.15 86.1128) (end 114.1419 80.1047) (width 0.25) (layer "F.Cu") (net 6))
 (segment (start 106.45 81.4001) (end 106.45 81.66) (width 0.25) (layer "F.Cu") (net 6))
 (segment (start 102.3465 89.2407) (end 102.3465 94.963) (width 0.25) (layer "F.Cu") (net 6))
 (segment (start 112.32 92.27) (end 112.32 91.1647) (width 0.25) (layer "F.Cu") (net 6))
 (segment (start 110.07 96.12) (end 108.9647 96.12) (width 0.25) (layer "F.Cu") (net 6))
 (segment (start 111.9455 91.1647) (end 112.32 91.1647) (width 0.25) (layer "F.Cu") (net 6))
 (segment (start 106.45 83.1723) (end 106.184 83.4383) (width 0.25) (layer "F.Cu") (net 6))
 (segment (start 97.55 110.46) (end 97.55 109.3047) (width 0.25) (layer "F.Cu") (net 6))
 (segment (start 102.3465 94.963) (end 103.7231 96.3396) (width 0.25) (layer "F.Cu") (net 6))
 (segment (start 106.184 85.4032) (end 111.9455 91.1647) (width 0.25) (layer "F.Cu") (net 6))
 (segment (start 97.8389 109.3047) (end 103.7231 103.4205) (width 0.25) (layer "F.Cu") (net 6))
 (segment (start 106.184 85.4032) (end 102.3465 89.2407) (width 0.25) (layer "F.Cu") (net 6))
 (segment (start 104.25 78.91) (end 104.25 76.8547) (width 0.25) (layer "B.Cu") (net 36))
 (segment (start 115.65 78.91) (end 115.65 76.8547) (width 0.25) (layer "B.Cu") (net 36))
 (segment (start 104.25 76.8547) (end 115.65 76.8547) (width 0.25) (layer "B.Cu") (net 36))
 (segment (start 114.32 106.68) (end 115.4753 106.68) (width 0.25) (layer "B.Cu") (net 34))
 (segment (start 118.66 106.66) (end 115.4953 106.66) (width 0.25) (layer "B.Cu") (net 34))
 (segment (start 115.4953 106.66) (end 115.4753 106.68) (width 0.25) (layer "B.Cu") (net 34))
 (segment (start 105.35 102.035) (end 105.725 102.41) (width 0.25) (layer "F.Cu") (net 32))
 (segment (start 105.35 99.29) (end 105.35 102.035) (width 0.25) (layer "F.Cu") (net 32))
 (segment (start 113.12 100.77) (end 113.12 101.8753) (width 0.25) (layer "F.Cu") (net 38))
 (segment (start 97.1118 111.6622) (end 103.3331 111.6622) (width 0.25) (layer "F.Cu") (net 38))
 (segment (start 103.3331 111.6622) (end 113.12 101.8753) (width 0.25) (layer "F.Cu") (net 38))
 (segment (start 97.55 107.92) (end 96.3869 109.0831) (width 0.25) (layer "F.Cu") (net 38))
 (segment (start 96.3869 110.9373) (end 97.1118 111.6622) (width 0.25) (layer "F.Cu") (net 38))
 (segment (start 96.3869 109.0831) (end 96.3869 110.9373) (width 0.25) (layer "F.Cu") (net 38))
 (segment (start 106.02 99.32) (end 105.99 99.29) (width 0.25) (layer "F.Cu") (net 10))
 (segment (start 110.07 99.32) (end 106.02 99.32) (width 0.25) (layer "F.Cu") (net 10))
 (segment (start 117.39 104.2482) (end 119.6753 101.9629) (width 0.25) (layer "F.Cu") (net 20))
 (segment (start 118.57 98.52) (end 119.6753 98.52) (width 0.25) (layer "F.Cu") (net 20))
 (segment (start 119.6753 101.9629) (end 119.6753 98.52) (width 0.25) (layer "F.Cu") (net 20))
 (segment (start 117.39 107.93) (end 117.39 104.2482) (width 0.25) (layer "F.Cu") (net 20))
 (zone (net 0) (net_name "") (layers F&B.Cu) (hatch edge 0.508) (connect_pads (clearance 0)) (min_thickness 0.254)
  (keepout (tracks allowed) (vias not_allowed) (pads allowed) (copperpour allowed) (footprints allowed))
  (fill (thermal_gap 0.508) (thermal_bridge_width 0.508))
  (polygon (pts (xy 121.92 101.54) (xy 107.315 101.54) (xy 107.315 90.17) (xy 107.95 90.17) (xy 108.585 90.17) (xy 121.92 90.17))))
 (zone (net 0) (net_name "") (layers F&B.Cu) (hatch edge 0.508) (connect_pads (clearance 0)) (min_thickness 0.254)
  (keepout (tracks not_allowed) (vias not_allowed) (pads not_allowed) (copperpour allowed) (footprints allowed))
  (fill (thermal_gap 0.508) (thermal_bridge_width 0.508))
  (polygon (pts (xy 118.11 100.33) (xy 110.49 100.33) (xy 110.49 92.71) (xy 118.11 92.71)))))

